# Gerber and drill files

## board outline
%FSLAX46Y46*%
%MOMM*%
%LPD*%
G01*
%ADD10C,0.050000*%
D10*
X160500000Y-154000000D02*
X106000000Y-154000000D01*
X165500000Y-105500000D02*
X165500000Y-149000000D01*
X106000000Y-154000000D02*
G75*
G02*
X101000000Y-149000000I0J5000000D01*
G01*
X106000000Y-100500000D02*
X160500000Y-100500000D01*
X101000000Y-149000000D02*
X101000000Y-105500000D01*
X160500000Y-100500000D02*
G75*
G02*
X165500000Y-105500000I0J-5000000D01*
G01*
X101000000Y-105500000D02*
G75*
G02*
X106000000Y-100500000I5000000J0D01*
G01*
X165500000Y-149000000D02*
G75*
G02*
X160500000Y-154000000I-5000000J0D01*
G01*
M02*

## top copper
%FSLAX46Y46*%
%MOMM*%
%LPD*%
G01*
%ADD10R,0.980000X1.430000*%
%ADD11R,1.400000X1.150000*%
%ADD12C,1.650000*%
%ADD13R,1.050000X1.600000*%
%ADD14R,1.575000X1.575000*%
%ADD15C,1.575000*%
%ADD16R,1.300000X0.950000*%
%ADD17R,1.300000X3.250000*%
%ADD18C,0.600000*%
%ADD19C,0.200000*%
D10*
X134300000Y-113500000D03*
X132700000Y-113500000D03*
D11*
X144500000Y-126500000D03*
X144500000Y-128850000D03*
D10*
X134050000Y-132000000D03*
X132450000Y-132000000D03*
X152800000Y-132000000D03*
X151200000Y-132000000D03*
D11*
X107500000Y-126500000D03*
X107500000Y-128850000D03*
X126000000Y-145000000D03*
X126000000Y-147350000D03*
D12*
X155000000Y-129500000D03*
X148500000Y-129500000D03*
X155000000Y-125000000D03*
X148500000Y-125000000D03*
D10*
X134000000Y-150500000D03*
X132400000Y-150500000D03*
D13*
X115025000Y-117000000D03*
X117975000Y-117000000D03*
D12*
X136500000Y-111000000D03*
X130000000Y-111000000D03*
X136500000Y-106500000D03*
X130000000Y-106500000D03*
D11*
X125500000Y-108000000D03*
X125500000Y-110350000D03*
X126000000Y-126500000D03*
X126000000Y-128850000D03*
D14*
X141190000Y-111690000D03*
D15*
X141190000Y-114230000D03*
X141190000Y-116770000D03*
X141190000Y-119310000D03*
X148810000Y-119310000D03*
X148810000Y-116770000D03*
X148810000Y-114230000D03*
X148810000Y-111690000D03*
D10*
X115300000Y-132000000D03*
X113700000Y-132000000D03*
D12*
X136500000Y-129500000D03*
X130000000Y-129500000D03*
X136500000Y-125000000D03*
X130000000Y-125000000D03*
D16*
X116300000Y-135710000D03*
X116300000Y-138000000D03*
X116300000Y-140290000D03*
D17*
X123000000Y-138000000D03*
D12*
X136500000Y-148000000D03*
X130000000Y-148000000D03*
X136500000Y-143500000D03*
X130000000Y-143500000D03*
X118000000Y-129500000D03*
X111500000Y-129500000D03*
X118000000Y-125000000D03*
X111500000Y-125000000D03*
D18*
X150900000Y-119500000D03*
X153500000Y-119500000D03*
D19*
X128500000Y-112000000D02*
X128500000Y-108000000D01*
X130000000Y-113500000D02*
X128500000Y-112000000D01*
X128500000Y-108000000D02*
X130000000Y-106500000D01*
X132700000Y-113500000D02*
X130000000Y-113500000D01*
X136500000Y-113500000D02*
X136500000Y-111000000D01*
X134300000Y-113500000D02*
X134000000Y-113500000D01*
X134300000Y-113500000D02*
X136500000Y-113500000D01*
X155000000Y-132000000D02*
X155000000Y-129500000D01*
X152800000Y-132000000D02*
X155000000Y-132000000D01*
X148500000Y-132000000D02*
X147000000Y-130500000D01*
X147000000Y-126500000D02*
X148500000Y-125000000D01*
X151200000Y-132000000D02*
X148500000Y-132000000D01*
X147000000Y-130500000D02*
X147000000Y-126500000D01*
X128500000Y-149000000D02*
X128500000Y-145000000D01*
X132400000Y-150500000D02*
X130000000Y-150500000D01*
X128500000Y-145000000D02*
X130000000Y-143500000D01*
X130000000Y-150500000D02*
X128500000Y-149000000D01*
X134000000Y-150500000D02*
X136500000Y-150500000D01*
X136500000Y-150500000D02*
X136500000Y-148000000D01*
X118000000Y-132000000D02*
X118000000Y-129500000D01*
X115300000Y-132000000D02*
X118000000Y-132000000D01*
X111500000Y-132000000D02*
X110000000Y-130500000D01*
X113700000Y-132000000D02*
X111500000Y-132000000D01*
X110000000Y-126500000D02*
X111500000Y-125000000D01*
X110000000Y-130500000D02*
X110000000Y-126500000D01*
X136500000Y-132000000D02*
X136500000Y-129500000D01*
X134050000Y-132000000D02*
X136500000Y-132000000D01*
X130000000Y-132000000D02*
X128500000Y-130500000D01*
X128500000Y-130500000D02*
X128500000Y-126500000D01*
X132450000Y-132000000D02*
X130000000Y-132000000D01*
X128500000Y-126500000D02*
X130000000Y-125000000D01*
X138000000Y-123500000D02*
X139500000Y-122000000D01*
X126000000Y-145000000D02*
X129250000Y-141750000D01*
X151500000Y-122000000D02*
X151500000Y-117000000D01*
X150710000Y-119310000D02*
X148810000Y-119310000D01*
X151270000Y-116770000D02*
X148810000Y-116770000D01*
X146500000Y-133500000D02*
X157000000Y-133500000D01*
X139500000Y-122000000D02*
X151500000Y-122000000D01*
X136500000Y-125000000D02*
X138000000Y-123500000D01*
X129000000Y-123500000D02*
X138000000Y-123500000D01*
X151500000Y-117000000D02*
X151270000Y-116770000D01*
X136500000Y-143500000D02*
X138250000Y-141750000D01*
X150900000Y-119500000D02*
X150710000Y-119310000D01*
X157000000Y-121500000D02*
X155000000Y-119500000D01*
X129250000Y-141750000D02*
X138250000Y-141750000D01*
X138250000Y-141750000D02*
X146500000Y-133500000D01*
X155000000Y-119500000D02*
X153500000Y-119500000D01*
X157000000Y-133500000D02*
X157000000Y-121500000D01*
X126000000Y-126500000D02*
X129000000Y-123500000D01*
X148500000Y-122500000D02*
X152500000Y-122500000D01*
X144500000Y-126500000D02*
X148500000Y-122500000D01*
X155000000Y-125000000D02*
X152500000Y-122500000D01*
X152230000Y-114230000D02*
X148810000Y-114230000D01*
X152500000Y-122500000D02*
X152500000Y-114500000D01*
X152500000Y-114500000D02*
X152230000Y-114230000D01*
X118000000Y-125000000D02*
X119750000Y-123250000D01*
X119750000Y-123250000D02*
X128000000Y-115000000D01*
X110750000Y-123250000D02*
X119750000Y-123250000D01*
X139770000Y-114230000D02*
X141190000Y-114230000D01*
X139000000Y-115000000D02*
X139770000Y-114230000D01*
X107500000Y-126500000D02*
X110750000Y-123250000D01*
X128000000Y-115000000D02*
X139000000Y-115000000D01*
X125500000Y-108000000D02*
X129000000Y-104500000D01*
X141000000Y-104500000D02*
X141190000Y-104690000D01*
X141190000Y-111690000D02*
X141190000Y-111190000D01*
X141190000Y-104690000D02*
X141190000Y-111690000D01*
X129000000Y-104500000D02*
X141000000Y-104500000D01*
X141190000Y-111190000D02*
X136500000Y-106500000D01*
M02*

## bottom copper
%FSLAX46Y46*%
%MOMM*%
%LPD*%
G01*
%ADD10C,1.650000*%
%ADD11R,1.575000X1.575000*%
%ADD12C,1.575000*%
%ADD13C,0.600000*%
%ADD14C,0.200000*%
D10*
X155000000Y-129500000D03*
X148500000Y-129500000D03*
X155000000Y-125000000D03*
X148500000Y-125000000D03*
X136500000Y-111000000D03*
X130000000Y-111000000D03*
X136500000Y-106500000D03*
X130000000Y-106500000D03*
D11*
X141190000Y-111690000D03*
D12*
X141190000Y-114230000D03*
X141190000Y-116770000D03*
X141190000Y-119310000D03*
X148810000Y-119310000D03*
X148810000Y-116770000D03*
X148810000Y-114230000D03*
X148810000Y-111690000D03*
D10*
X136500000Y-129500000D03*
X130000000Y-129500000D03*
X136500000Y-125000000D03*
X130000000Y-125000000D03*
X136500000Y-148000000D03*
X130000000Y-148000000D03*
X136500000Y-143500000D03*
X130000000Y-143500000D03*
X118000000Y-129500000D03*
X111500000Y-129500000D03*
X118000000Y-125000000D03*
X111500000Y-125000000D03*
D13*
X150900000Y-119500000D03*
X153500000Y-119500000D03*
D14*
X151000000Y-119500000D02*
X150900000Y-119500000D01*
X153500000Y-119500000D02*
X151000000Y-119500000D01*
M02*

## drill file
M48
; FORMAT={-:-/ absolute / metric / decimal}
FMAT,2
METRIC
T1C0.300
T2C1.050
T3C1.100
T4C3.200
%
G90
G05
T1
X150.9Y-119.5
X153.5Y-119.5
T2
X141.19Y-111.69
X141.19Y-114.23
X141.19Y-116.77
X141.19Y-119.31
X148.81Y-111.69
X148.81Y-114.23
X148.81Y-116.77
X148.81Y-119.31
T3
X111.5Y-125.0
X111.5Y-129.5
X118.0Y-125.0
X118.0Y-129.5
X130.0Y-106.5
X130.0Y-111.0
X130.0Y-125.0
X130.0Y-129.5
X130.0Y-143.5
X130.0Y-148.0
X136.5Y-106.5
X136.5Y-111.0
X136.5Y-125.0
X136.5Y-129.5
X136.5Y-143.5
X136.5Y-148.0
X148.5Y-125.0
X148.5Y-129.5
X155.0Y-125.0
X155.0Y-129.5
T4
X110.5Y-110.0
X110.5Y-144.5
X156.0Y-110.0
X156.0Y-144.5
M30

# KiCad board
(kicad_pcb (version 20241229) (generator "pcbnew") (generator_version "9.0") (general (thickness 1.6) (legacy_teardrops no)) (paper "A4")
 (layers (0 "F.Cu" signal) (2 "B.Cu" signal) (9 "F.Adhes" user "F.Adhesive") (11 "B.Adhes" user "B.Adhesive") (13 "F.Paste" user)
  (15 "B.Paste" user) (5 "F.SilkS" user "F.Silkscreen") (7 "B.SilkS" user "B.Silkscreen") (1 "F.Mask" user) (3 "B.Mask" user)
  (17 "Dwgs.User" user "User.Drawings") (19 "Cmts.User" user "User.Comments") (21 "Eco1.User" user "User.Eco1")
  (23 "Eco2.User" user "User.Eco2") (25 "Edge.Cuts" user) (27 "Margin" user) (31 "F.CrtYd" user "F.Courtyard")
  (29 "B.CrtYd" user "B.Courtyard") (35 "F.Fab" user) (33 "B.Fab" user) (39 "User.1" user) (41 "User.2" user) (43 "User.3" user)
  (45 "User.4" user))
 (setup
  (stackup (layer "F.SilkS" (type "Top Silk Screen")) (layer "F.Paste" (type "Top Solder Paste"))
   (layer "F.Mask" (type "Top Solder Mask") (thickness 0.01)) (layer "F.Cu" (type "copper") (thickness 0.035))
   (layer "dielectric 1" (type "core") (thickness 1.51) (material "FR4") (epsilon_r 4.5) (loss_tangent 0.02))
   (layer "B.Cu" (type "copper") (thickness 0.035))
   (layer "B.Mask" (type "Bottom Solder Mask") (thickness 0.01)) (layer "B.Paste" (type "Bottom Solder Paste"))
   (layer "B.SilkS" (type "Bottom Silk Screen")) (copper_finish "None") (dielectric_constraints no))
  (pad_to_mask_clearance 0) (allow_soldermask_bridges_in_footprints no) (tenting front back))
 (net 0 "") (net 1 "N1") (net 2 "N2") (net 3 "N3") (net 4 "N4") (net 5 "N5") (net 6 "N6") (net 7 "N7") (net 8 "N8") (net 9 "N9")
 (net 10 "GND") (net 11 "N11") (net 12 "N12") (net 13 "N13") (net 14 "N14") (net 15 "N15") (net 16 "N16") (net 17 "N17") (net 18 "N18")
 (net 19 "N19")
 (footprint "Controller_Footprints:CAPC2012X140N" (layer "F.Cu") (at 133.5 113.5 180)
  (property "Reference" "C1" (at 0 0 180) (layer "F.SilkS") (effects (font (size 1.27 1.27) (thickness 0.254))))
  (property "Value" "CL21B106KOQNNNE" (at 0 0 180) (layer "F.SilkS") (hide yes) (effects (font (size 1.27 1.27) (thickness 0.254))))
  (pad "1" smd rect (at -0.8 0 180) (size 0.98 1.43) (layers "F.Cu" "F.Mask" "F.Paste") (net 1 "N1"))
  (pad "2" smd rect (at 0.8 0 180) (size 0.98 1.43) (layers "F.Cu" "F.Mask" "F.Paste") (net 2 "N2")))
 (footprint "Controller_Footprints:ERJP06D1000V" (layer "F.Cu") (at 144.5 127.675 -90)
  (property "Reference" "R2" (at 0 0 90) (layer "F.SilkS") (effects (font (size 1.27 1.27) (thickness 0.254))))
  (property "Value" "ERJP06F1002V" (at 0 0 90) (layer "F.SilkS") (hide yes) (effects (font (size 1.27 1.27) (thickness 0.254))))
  (pad "1" smd rect (at -1.175 0 270) (size 1.15 1.4) (layers "F.Cu" "F.Mask" "F.Paste") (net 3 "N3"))
  (pad "2" smd rect (at 1.175 0 270) (size 1.15 1.4) (layers "F.Cu" "F.Mask" "F.Paste") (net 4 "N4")))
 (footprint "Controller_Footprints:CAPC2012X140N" (layer "F.Cu") (at 133.25 132 180)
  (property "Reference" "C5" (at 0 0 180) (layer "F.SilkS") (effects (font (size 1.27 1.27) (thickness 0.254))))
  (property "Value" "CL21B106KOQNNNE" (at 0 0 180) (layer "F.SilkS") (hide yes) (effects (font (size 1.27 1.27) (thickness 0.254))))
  (pad "1" smd rect (at -0.8 0 180) (size 0.98 1.43) (layers "F.Cu" "F.Mask" "F.Paste") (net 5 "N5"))
  (pad "2" smd rect (at 0.8 0 180) (size 0.98 1.43) (layers "F.Cu" "F.Mask" "F.Paste") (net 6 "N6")))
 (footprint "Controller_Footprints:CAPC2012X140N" (layer "F.Cu") (at 152 132 180)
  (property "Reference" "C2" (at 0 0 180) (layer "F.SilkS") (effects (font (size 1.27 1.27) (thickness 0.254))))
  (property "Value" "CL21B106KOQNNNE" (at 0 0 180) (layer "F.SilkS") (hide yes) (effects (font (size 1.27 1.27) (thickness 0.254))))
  (pad "1" smd rect (at -0.8 0 180) (size 0.98 1.43) (layers "F.Cu" "F.Mask" "F.Paste") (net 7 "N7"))
  (pad "2" smd rect (at 0.8 0 180) (size 0.98 1.43) (layers "F.Cu" "F.Mask" "F.Paste") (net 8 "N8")))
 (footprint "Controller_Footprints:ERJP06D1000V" (layer "F.Cu") (at 107.5 127.675 -90)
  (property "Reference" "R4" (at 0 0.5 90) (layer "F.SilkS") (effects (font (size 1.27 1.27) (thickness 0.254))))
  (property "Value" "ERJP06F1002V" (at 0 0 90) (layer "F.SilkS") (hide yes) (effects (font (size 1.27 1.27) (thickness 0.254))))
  (pad "1" smd rect (at -1.175 0 270) (size 1.15 1.4) (layers "F.Cu" "F.Mask" "F.Paste") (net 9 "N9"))
  (pad "2" smd rect (at 1.175 0 270) (size 1.15 1.4) (layers "F.Cu" "F.Mask" "F.Paste") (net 4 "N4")))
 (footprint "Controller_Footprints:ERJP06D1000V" (layer "F.Cu") (at 126 146.175 -90)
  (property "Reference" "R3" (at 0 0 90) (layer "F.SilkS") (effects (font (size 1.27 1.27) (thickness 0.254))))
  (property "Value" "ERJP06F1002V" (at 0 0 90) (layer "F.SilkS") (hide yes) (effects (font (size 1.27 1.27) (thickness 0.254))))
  (pad "1" smd rect (at -1.175 0 270) (size 1.15 1.4) (layers "F.Cu" "F.Mask" "F.Paste") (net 4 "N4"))
  (pad "2" smd rect (at 1.175 0 270) (size 1.15 1.4) (layers "F.Cu" "F.Mask" "F.Paste") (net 4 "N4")))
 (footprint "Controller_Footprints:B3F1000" (layer "F.Cu") (at 151.75 127.25)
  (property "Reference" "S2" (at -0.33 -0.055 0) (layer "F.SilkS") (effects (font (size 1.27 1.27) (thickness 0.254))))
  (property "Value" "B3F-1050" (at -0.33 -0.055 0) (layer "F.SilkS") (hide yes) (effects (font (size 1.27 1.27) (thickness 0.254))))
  (pad "1" thru_hole circle (at 3.25 2.25) (size 1.65 1.65) (drill 1.1) (layers "*.Cu" "*.Mask") (remove_unused_layers no) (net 7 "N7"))
  (pad "2" thru_hole circle (at -3.25 2.25) (size 1.65 1.65) (drill 1.1) (layers "*.Cu" "*.Mask") (remove_unused_layers no) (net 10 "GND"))
  (pad "3" thru_hole circle (at 3.25 -2.25) (size 1.65 1.65) (drill 1.1) (layers "*.Cu" "*.Mask") (remove_unused_layers no) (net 4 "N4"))
  (pad "4" thru_hole circle (at -3.25 -2.25) (size 1.65 1.65) (drill 1.1) (layers "*.Cu" "*.Mask") (remove_unused_layers no) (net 8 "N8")))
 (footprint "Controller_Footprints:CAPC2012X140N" (layer "F.Cu") (at 133.2 150.5 180)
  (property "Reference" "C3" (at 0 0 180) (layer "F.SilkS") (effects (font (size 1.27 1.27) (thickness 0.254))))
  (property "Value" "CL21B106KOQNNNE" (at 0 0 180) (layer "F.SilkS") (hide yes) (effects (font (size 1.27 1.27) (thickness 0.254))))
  (pad "1" smd rect (at -0.8 0 180) (size 0.98 1.43) (layers "F.Cu" "F.Mask" "F.Paste") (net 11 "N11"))
  (pad "2" smd rect (at 0.8 0 180) (size 0.98 1.43) (layers "F.Cu" "F.Mask" "F.Paste") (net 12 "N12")))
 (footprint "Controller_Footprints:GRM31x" (layer "F.Cu") (at 116.5 117)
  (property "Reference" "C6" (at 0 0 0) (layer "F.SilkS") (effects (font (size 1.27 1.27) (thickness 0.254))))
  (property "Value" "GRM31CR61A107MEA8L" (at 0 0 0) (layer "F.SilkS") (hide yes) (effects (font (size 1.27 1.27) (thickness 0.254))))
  (pad "1" smd rect (at -1.475 0) (size 1.05 1.6) (layers "F.Cu" "F.Mask" "F.Paste") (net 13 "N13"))
  (pad "2" smd rect (at 1.475 0) (size 1.05 1.6) (layers "F.Cu" "F.Mask" "F.Paste") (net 10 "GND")))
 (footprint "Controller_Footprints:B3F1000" (layer "F.Cu") (at 133.25 108.75)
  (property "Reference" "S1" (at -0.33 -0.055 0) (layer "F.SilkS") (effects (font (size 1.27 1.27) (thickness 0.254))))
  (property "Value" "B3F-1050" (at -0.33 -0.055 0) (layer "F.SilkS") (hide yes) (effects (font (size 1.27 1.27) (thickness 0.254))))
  (pad "1" thru_hole circle (at 3.25 2.25) (size 1.65 1.65) (drill 1.1) (layers "*.Cu" "*.Mask") (remove_unused_layers no) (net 1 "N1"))
  (pad "2" thru_hole circle (at -3.25 2.25) (size 1.65 1.65) (drill 1.1) (layers "*.Cu" "*.Mask") (remove_unused_layers no) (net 10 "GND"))
  (pad "3" thru_hole circle (at 3.25 -2.25) (size 1.65 1.65) (drill 1.1) (layers "*.Cu" "*.Mask") (remove_unused_layers no) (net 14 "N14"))
  (pad "4" thru_hole circle (at -3.25 -2.25) (size 1.65 1.65) (drill 1.1) (layers "*.Cu" "*.Mask") (remove_unused_layers no) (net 2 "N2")))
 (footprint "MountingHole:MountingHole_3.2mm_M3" (layer "F.Cu") (at 110.5 110)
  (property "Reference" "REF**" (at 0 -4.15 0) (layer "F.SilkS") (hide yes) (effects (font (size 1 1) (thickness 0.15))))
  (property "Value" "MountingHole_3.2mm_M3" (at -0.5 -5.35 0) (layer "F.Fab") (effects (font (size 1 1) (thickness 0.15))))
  (pad "" np_thru_hole circle (at 0 0) (size 3.2 3.2) (drill 3.2) (layers "*.Cu" "*.Mask")))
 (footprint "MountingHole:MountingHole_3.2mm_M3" (layer "F.Cu") (at 110.5 144.5)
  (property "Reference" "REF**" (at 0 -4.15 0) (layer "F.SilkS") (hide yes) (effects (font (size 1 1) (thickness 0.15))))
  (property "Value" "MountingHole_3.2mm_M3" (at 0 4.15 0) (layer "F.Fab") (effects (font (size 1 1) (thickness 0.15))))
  (pad "" np_thru_hole circle (at 0 0) (size 3.2 3.2) (drill 3.2) (layers "*.Cu" "*.Mask")))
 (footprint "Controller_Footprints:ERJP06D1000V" (layer "F.Cu") (at 125.5 109.175 -90)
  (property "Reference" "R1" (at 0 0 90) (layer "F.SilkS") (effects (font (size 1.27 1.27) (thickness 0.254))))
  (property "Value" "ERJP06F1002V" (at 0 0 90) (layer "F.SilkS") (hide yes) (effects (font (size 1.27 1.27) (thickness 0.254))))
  (pad "1" smd rect (at -1.175 0 270) (size 1.15 1.4) (layers "F.Cu" "F.Mask" "F.Paste") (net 14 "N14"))
  (pad "2" smd rect (at 1.175 0 270) (size 1.15 1.4) (layers "F.Cu" "F.Mask" "F.Paste") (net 4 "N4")))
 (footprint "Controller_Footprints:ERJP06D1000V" (layer "F.Cu") (at 126 127.675 -90)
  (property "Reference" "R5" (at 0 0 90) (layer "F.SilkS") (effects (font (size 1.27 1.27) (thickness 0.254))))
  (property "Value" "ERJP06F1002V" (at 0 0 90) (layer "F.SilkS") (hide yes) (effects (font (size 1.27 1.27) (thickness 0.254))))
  (pad "1" smd rect (at -1.175 0 270) (size 1.15 1.4) (layers "F.Cu" "F.Mask" "F.Paste") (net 4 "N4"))
  (pad "2" smd rect (at 1.175 0 270) (size 1.15 1.4) (layers "F.Cu" "F.Mask" "F.Paste") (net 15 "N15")))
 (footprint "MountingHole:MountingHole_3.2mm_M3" (layer "F.Cu") (at 156 144.5)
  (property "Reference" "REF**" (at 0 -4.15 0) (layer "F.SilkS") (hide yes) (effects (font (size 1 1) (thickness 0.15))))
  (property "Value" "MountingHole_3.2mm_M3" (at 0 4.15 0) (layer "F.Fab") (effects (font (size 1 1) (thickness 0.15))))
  (pad "" np_thru_hole circle (at 0 0) (size 3.2 3.2) (drill 3.2) (layers "*.Cu" "*.Mask")))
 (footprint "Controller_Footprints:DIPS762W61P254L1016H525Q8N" (layer "F.Cu") (at 141.19 111.69)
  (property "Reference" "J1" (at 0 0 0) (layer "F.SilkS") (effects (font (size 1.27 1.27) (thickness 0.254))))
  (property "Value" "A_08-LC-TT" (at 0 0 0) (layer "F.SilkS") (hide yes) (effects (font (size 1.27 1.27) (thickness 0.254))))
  (pad "1" thru_hole rect (at 0 0) (size 1.575 1.575) (drill 1.05) (layers "*.Cu" "*.Mask") (remove_unused_layers no) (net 14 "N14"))
  (pad "2" thru_hole circle (at 0 2.54) (size 1.575 1.575) (drill 1.05) (layers "*.Cu" "*.Mask") (remove_unused_layers no) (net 9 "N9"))
  (pad "3" thru_hole circle (at 0 5.08) (size 1.575 1.575) (drill 1.05) (layers "*.Cu" "*.Mask") (remove_unused_layers no) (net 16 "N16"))
  (pad "4" thru_hole circle (at 0 7.62) (size 1.575 1.575) (drill 1.05) (layers "*.Cu" "*.Mask") (remove_unused_layers no) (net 10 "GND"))
  (pad "5" thru_hole circle (at 7.62 7.62) (size 1.575 1.575) (drill 1.05) (layers "*.Cu" "*.Mask") (remove_unused_layers no) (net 4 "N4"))
  (pad "6" thru_hole circle (at 7.62 5.08) (size 1.575 1.575) (drill 1.05) (layers "*.Cu" "*.Mask") (remove_unused_layers no) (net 15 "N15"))
  (pad "7" thru_hole circle (at 7.62 2.54) (size 1.575 1.575) (drill 1.05) (layers "*.Cu" "*.Mask") (remove_unused_layers no) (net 3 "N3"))
  (pad "8" thru_hole circle (at 7.62 0) (size 1.575 1.575) (drill 1.05) (layers "*.Cu" "*.Mask") (remove_unused_layers no) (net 4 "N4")))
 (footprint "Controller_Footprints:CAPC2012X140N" (layer "F.Cu") (at 114.5 132 180)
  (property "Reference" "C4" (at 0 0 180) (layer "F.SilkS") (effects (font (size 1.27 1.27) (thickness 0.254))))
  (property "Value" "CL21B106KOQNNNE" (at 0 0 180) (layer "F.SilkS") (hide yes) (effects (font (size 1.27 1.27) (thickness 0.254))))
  (pad "1" smd rect (at -0.8 0 180) (size 0.98 1.43) (layers "F.Cu" "F.Mask" "F.Paste") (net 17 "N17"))
  (pad "2" smd rect (at 0.8 0 180) (size 0.98 1.43) (layers "F.Cu" "F.Mask" "F.Paste") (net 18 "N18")))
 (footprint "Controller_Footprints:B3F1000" (layer "F.Cu") (at 133.25 127.25)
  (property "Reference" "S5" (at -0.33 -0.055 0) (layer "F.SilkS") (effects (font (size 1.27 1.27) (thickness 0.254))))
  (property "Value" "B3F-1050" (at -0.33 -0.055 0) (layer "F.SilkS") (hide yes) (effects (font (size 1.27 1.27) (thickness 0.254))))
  (pad "1" thru_hole circle (at 3.25 2.25) (size 1.65 1.65) (drill 1.1) (layers "*.Cu" "*.Mask") (remove_unused_layers no) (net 5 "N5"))
  (pad "2" thru_hole circle (at -3.25 2.25) (size 1.65 1.65) (drill 1.1) (layers "*.Cu" "*.Mask") (remove_unused_layers no) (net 10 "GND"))
  (pad "3" thru_hole circle (at 3.25 -2.25) (size 1.65 1.65) (drill 1.1) (layers "*.Cu" "*.Mask") (remove_unused_layers no) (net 4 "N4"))
  (pad "4" thru_hole circle (at -3.25 -2.25) (size 1.65 1.65) (drill 1.1) (layers "*.Cu" "*.Mask") (remove_unused_layers no) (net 6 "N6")))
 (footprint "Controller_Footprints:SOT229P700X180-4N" (layer "F.Cu") (at 119.65 138)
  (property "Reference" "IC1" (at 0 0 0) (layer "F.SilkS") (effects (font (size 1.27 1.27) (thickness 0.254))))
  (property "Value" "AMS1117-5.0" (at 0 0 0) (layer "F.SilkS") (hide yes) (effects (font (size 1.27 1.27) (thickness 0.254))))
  (pad "1" smd rect (at -3.35 -2.29 90) (size 0.95 1.3) (layers "F.Cu" "F.Mask" "F.Paste") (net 10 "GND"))
  (pad "2" smd rect (at -3.35 0 90) (size 0.95 1.3) (layers "F.Cu" "F.Mask" "F.Paste") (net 4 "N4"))
  (pad "3" smd rect (at -3.35 2.29 90) (size 0.95 1.3) (layers "F.Cu" "F.Mask" "F.Paste") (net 13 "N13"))
  (pad "4" smd rect (at 3.35 0) (size 1.3 3.25) (layers "F.Cu" "F.Mask" "F.Paste") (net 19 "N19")))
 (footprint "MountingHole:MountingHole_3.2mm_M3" (layer "F.Cu") (at 156 110)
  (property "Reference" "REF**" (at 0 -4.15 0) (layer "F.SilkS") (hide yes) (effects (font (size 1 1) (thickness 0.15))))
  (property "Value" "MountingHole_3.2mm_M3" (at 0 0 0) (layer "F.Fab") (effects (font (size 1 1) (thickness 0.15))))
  (pad "" np_thru_hole circle (at 0 0) (size 3.2 3.2) (drill 3.2) (layers "*.Cu" "*.Mask")))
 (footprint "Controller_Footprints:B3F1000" (layer "F.Cu") (at 133.25 145.75)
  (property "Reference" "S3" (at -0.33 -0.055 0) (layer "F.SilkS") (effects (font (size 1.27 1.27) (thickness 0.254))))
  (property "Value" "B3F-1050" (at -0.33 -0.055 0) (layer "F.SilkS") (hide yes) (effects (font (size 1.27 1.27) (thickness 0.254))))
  (pad "1" thru_hole circle (at 3.25 2.25) (size 1.65 1.65) (drill 1.1) (layers "*.Cu" "*.Mask") (remove_unused_layers no) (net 11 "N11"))
  (pad "2" thru_hole circle (at -3.25 2.25) (size 1.65 1.65) (drill 1.1) (layers "*.Cu" "*.Mask") (remove_unused_layers no) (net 10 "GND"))
  (pad "3" thru_hole circle (at 3.25 -2.25) (size 1.65 1.65) (drill 1.1) (layers "*.Cu" "*.Mask") (remove_unused_layers no) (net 4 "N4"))
  (pad "4" thru_hole circle (at -3.25 -2.25) (size 1.65 1.65) (drill 1.1) (layers "*.Cu" "*.Mask") (remove_unused_layers no) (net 12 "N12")))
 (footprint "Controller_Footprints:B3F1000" (layer "F.Cu") (at 114.75 127.25)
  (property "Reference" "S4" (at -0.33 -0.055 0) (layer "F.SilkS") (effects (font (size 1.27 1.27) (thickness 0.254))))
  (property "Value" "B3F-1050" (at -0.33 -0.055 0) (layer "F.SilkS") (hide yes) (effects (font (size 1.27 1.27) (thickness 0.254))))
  (pad "1" thru_hole circle (at 3.25 2.25) (size 1.65 1.65) (drill 1.1) (layers "*.Cu" "*.Mask") (remove_unused_layers no) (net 17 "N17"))
  (pad "2" thru_hole circle (at -3.25 2.25) (size 1.65 1.65) (drill 1.1) (layers "*.Cu" "*.Mask") (remove_unused_layers no) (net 10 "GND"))
  (pad "3" thru_hole circle (at 3.25 -2.25) (size 1.65 1.65) (drill 1.1) (layers "*.Cu" "*.Mask") (remove_unused_layers no) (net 9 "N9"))
  (pad "4" thru_hole circle (at -3.25 -2.25) (size 1.65 1.65) (drill 1.1) (layers "*.Cu" "*.Mask") (remove_unused_layers no) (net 18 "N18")))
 (gr_line (start 160.5 154) (end 106 154) (stroke (width 0.05) (type default)) (layer "Edge.Cuts"))
 (gr_line (start 165.5 105.5) (end 165.5 149) (stroke (width 0.05) (type default)) (layer "Edge.Cuts"))
 (gr_arc (start 106 154) (mid 102.464466 152.535534) (end 101 149) (stroke (width 0.05) (type default)) (layer "Edge.Cuts"))
 (gr_line (start 106 100.5) (end 160.5 100.5) (stroke (width 0.05) (type default)) (layer "Edge.Cuts"))
 (gr_line (start 101 149) (end 101 105.5) (stroke (width 0.05) (type default)) (layer "Edge.Cuts"))
 (gr_arc (start 160.5 100.5) (mid 164.035534 101.964466) (end 165.5 105.5) (stroke (width 0.05) (type default)) (layer "Edge.Cuts"))
 (gr_arc (start 101 105.5) (mid 102.464466 101.964466) (end 106 100.5) (stroke (width 0.05) (type default)) (layer "Edge.Cuts"))
 (gr_arc (start 165.5 149) (mid 164.035534 152.535534) (end 160.5 154) (stroke (width 0.05) (type default)) (layer "Edge.Cuts"))
 (segment (start 128.5 112) (end 128.5 108) (width 0.2) (layer "F.Cu") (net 2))
 (segment (start 130 113.5) (end 128.5 112) (width 0.2) (layer "F.Cu") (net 2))
 (segment (start 128.5 108) (end 130 106.5) (width 0.2) (layer "F.Cu") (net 2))
 (segment (start 132.7 113.5) (end 130 113.5) (width 0.2) (layer "F.Cu") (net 2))
 (segment (start 136.5 113.5) (end 136.5 111) (width 0.2) (layer "F.Cu") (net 1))
 (segment (start 134.3 113.5) (end 134 113.5) (width 0.2) (layer "F.Cu") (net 1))
 (segment (start 134.3 113.5) (end 136.5 113.5) (width 0.2) (layer "F.Cu") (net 1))
 (segment (start 155 132) (end 155 129.5) (width 0.2) (layer "F.Cu") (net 7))
 (segment (start 152.8 132) (end 155 132) (width 0.2) (layer "F.Cu") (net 7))
 (segment (start 148.5 132) (end 147 130.5) (width 0.2) (layer "F.Cu") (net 8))
 (segment (start 147 126.5) (end 148.5 125) (width 0.2) (layer "F.Cu") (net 8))
 (segment (start 151.2 132) (end 148.5 132) (width 0.2) (layer "F.Cu") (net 8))
 (segment (start 147 130.5) (end 147 126.5) (width 0.2) (layer "F.Cu") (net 8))
 (segment (start 128.5 149) (end 128.5 145) (width 0.2) (layer "F.Cu") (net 12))
 (segment (start 132.4 150.5) (end 130 150.5) (width 0.2) (layer "F.Cu") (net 12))
 (segment (start 128.5 145) (end 130 143.5) (width 0.2) (layer "F.Cu") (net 12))
 (segment (start 130 150.5) (end 128.5 149) (width 0.2) (layer "F.Cu") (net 12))
 (segment (start 134 150.5) (end 136.5 150.5) (width 0.2) (layer "F.Cu") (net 11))
 (segment (start 136.5 150.5) (end 136.5 148) (width 0.2) (layer "F.Cu") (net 11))
 (segment (start 118 132) (end 118 129.5) (width 0.2) (layer "F.Cu") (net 17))
 (segment (start 115.3 132) (end 118 132) (width 0.2) (layer "F.Cu") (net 17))
 (segment (start 111.5 132) (end 110 130.5) (width 0.2) (layer "F.Cu") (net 18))
 (segment (start 113.7 132) (end 111.5 132) (width 0.2) (layer "F.Cu") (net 18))
 (segment (start 110 126.5) (end 111.5 125) (width 0.2) (layer "F.Cu") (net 18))
 (segment (start 110 130.5) (end 110 126.5) (width 0.2) (layer "F.Cu") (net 18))
 (segment (start 136.5 132) (end 136.5 129.5) (width 0.2) (layer "F.Cu") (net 5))
 (segment (start 134.05 132) (end 136.5 132) (width 0.2) (layer "F.Cu") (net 5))
 (segment (start 130 132) (end 128.5 130.5) (width 0.2) (layer "F.Cu") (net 6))
 (segment (start 128.5 130.5) (end 128.5 126.5) (width 0.2) (layer "F.Cu") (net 6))
 (segment (start 132.45 132) (end 130 132) (width 0.2) (layer "F.Cu") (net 6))
 (segment (start 128.5 126.5) (end 130 125) (width 0.2) (layer "F.Cu") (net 6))
 (segment (start 138 123.5) (end 139.5 122) (width 0.2) (layer "F.Cu") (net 4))
 (segment (start 126 145) (end 129.25 141.75) (width 0.2) (layer "F.Cu") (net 4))
 (segment (start 151.5 122) (end 151.5 117) (width 0.2) (layer "F.Cu") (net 4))
 (segment (start 150.71 119.31) (end 148.81 119.31) (width 0.2) (layer "F.Cu") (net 4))
 (segment (start 151.27 116.77) (end 148.81 116.77) (width 0.2) (layer "F.Cu") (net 4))
 (segment (start 146.5 133.5) (end 157 133.5) (width 0.2) (layer "F.Cu") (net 4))
 (segment (start 139.5 122) (end 151.5 122) (width 0.2) (layer "F.Cu") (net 4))
 (segment (start 136.5 125) (end 138 123.5) (width 0.2) (layer "F.Cu") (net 4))
 (segment (start 129 123.5) (end 138 123.5) (width 0.2) (layer "F.Cu") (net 4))
 (segment (start 151.5 117) (end 151.27 116.77) (width 0.2) (layer "F.Cu") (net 4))
 (segment (start 136.5 143.5) (end 138.25 141.75) (width 0.2) (layer "F.Cu") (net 4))
 (segment (start 150.9 119.5) (end 150.71 119.31) (width 0.2) (layer "F.Cu") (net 4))
 (segment (start 157 121.5) (end 155 119.5) (width 0.2) (layer "F.Cu") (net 4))
 (segment (start 129.25 141.75) (end 138.25 141.75) (width 0.2) (layer "F.Cu") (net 4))
 (segment (start 138.25 141.75) (end 146.5 133.5) (width 0.2) (layer "F.Cu") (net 4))
 (segment (start 155 119.5) (end 153.5 119.5) (width 0.2) (layer "F.Cu") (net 4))
 (segment (start 157 133.5) (end 157 121.5) (width 0.2) (layer "F.Cu") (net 4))
 (segment (start 126 126.5) (end 129 123.5) (width 0.2) (layer "F.Cu") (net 4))
 (via (at 150.9 119.5) (size 0.6) (drill 0.3) (layers "F.Cu" "B.Cu") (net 4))
 (via (at 153.5 119.5) (size 0.6) (drill 0.3) (layers "F.Cu" "B.Cu") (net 4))
 (segment (start 151 119.5) (end 150.9 119.5) (width 0.2) (layer "B.Cu") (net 4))
 (segment (start 153.5 119.5) (end 151 119.5) (width 0.2) (layer "B.Cu") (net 4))
 (segment (start 148.5 122.5) (end 152.5 122.5) (width 0.2) (layer "F.Cu") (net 3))
 (segment (start 144.5 126.5) (end 148.5 122.5) (width 0.2) (layer "F.Cu") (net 3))
 (segment (start 155 125) (end 152.5 122.5) (width 0.2) (layer "F.Cu") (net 3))
 (segment (start 152.23 114.23) (end 148.81 114.23) (width 0.2) (layer "F.Cu") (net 3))
 (segment (start 152.5 122.5) (end 152.5 114.5) (width 0.2) (layer "F.Cu") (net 3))
 (segment (start 152.5 114.5) (end 152.23 114.23) (width 0.2) (layer "F.Cu") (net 3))
 (segment (start 118 125) (end 119.75 123.25) (width 0.2) (layer "F.Cu") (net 9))
 (segment (start 119.75 123.25) (end 128 115) (width 0.2) (layer "F.Cu") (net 9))
 (segment (start 110.75 123.25) (end 119.75 123.25) (width 0.2) (layer "F.Cu") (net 9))
 (segment (start 139.77 114.23) (end 141.19 114.23) (width 0.2) (layer "F.Cu") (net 9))
 (segment (start 139 115) (end 139.77 114.23) (width 0.2) (layer "F.Cu") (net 9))
 (segment (start 107.5 126.5) (end 110.75 123.25) (width 0.2) (layer "F.Cu") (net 9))
 (segment (start 128 115) (end 139 115) (width 0.2) (layer "F.Cu") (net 9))
 (segment (start 125.5 108) (end 129 104.5) (width 0.2) (layer "F.Cu") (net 14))
 (segment (start 141 104.5) (end 141.19 104.69) (width 0.2) (layer "F.Cu") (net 14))
 (segment (start 141.19 111.69) (end 141.19 111.19) (width 0.2) (layer "F.Cu") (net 14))
 (segment (start 141.19 104.69) (end 141.19 111.69) (width 0.2) (layer "F.Cu") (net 14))
 (segment (start 129 104.5) (end 141 104.5) (width 0.2) (layer "F.Cu") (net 14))
 (segment (start 141.19 111.19) (end 136.5 106.5) (width 0.2) (layer "F.Cu") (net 14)))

